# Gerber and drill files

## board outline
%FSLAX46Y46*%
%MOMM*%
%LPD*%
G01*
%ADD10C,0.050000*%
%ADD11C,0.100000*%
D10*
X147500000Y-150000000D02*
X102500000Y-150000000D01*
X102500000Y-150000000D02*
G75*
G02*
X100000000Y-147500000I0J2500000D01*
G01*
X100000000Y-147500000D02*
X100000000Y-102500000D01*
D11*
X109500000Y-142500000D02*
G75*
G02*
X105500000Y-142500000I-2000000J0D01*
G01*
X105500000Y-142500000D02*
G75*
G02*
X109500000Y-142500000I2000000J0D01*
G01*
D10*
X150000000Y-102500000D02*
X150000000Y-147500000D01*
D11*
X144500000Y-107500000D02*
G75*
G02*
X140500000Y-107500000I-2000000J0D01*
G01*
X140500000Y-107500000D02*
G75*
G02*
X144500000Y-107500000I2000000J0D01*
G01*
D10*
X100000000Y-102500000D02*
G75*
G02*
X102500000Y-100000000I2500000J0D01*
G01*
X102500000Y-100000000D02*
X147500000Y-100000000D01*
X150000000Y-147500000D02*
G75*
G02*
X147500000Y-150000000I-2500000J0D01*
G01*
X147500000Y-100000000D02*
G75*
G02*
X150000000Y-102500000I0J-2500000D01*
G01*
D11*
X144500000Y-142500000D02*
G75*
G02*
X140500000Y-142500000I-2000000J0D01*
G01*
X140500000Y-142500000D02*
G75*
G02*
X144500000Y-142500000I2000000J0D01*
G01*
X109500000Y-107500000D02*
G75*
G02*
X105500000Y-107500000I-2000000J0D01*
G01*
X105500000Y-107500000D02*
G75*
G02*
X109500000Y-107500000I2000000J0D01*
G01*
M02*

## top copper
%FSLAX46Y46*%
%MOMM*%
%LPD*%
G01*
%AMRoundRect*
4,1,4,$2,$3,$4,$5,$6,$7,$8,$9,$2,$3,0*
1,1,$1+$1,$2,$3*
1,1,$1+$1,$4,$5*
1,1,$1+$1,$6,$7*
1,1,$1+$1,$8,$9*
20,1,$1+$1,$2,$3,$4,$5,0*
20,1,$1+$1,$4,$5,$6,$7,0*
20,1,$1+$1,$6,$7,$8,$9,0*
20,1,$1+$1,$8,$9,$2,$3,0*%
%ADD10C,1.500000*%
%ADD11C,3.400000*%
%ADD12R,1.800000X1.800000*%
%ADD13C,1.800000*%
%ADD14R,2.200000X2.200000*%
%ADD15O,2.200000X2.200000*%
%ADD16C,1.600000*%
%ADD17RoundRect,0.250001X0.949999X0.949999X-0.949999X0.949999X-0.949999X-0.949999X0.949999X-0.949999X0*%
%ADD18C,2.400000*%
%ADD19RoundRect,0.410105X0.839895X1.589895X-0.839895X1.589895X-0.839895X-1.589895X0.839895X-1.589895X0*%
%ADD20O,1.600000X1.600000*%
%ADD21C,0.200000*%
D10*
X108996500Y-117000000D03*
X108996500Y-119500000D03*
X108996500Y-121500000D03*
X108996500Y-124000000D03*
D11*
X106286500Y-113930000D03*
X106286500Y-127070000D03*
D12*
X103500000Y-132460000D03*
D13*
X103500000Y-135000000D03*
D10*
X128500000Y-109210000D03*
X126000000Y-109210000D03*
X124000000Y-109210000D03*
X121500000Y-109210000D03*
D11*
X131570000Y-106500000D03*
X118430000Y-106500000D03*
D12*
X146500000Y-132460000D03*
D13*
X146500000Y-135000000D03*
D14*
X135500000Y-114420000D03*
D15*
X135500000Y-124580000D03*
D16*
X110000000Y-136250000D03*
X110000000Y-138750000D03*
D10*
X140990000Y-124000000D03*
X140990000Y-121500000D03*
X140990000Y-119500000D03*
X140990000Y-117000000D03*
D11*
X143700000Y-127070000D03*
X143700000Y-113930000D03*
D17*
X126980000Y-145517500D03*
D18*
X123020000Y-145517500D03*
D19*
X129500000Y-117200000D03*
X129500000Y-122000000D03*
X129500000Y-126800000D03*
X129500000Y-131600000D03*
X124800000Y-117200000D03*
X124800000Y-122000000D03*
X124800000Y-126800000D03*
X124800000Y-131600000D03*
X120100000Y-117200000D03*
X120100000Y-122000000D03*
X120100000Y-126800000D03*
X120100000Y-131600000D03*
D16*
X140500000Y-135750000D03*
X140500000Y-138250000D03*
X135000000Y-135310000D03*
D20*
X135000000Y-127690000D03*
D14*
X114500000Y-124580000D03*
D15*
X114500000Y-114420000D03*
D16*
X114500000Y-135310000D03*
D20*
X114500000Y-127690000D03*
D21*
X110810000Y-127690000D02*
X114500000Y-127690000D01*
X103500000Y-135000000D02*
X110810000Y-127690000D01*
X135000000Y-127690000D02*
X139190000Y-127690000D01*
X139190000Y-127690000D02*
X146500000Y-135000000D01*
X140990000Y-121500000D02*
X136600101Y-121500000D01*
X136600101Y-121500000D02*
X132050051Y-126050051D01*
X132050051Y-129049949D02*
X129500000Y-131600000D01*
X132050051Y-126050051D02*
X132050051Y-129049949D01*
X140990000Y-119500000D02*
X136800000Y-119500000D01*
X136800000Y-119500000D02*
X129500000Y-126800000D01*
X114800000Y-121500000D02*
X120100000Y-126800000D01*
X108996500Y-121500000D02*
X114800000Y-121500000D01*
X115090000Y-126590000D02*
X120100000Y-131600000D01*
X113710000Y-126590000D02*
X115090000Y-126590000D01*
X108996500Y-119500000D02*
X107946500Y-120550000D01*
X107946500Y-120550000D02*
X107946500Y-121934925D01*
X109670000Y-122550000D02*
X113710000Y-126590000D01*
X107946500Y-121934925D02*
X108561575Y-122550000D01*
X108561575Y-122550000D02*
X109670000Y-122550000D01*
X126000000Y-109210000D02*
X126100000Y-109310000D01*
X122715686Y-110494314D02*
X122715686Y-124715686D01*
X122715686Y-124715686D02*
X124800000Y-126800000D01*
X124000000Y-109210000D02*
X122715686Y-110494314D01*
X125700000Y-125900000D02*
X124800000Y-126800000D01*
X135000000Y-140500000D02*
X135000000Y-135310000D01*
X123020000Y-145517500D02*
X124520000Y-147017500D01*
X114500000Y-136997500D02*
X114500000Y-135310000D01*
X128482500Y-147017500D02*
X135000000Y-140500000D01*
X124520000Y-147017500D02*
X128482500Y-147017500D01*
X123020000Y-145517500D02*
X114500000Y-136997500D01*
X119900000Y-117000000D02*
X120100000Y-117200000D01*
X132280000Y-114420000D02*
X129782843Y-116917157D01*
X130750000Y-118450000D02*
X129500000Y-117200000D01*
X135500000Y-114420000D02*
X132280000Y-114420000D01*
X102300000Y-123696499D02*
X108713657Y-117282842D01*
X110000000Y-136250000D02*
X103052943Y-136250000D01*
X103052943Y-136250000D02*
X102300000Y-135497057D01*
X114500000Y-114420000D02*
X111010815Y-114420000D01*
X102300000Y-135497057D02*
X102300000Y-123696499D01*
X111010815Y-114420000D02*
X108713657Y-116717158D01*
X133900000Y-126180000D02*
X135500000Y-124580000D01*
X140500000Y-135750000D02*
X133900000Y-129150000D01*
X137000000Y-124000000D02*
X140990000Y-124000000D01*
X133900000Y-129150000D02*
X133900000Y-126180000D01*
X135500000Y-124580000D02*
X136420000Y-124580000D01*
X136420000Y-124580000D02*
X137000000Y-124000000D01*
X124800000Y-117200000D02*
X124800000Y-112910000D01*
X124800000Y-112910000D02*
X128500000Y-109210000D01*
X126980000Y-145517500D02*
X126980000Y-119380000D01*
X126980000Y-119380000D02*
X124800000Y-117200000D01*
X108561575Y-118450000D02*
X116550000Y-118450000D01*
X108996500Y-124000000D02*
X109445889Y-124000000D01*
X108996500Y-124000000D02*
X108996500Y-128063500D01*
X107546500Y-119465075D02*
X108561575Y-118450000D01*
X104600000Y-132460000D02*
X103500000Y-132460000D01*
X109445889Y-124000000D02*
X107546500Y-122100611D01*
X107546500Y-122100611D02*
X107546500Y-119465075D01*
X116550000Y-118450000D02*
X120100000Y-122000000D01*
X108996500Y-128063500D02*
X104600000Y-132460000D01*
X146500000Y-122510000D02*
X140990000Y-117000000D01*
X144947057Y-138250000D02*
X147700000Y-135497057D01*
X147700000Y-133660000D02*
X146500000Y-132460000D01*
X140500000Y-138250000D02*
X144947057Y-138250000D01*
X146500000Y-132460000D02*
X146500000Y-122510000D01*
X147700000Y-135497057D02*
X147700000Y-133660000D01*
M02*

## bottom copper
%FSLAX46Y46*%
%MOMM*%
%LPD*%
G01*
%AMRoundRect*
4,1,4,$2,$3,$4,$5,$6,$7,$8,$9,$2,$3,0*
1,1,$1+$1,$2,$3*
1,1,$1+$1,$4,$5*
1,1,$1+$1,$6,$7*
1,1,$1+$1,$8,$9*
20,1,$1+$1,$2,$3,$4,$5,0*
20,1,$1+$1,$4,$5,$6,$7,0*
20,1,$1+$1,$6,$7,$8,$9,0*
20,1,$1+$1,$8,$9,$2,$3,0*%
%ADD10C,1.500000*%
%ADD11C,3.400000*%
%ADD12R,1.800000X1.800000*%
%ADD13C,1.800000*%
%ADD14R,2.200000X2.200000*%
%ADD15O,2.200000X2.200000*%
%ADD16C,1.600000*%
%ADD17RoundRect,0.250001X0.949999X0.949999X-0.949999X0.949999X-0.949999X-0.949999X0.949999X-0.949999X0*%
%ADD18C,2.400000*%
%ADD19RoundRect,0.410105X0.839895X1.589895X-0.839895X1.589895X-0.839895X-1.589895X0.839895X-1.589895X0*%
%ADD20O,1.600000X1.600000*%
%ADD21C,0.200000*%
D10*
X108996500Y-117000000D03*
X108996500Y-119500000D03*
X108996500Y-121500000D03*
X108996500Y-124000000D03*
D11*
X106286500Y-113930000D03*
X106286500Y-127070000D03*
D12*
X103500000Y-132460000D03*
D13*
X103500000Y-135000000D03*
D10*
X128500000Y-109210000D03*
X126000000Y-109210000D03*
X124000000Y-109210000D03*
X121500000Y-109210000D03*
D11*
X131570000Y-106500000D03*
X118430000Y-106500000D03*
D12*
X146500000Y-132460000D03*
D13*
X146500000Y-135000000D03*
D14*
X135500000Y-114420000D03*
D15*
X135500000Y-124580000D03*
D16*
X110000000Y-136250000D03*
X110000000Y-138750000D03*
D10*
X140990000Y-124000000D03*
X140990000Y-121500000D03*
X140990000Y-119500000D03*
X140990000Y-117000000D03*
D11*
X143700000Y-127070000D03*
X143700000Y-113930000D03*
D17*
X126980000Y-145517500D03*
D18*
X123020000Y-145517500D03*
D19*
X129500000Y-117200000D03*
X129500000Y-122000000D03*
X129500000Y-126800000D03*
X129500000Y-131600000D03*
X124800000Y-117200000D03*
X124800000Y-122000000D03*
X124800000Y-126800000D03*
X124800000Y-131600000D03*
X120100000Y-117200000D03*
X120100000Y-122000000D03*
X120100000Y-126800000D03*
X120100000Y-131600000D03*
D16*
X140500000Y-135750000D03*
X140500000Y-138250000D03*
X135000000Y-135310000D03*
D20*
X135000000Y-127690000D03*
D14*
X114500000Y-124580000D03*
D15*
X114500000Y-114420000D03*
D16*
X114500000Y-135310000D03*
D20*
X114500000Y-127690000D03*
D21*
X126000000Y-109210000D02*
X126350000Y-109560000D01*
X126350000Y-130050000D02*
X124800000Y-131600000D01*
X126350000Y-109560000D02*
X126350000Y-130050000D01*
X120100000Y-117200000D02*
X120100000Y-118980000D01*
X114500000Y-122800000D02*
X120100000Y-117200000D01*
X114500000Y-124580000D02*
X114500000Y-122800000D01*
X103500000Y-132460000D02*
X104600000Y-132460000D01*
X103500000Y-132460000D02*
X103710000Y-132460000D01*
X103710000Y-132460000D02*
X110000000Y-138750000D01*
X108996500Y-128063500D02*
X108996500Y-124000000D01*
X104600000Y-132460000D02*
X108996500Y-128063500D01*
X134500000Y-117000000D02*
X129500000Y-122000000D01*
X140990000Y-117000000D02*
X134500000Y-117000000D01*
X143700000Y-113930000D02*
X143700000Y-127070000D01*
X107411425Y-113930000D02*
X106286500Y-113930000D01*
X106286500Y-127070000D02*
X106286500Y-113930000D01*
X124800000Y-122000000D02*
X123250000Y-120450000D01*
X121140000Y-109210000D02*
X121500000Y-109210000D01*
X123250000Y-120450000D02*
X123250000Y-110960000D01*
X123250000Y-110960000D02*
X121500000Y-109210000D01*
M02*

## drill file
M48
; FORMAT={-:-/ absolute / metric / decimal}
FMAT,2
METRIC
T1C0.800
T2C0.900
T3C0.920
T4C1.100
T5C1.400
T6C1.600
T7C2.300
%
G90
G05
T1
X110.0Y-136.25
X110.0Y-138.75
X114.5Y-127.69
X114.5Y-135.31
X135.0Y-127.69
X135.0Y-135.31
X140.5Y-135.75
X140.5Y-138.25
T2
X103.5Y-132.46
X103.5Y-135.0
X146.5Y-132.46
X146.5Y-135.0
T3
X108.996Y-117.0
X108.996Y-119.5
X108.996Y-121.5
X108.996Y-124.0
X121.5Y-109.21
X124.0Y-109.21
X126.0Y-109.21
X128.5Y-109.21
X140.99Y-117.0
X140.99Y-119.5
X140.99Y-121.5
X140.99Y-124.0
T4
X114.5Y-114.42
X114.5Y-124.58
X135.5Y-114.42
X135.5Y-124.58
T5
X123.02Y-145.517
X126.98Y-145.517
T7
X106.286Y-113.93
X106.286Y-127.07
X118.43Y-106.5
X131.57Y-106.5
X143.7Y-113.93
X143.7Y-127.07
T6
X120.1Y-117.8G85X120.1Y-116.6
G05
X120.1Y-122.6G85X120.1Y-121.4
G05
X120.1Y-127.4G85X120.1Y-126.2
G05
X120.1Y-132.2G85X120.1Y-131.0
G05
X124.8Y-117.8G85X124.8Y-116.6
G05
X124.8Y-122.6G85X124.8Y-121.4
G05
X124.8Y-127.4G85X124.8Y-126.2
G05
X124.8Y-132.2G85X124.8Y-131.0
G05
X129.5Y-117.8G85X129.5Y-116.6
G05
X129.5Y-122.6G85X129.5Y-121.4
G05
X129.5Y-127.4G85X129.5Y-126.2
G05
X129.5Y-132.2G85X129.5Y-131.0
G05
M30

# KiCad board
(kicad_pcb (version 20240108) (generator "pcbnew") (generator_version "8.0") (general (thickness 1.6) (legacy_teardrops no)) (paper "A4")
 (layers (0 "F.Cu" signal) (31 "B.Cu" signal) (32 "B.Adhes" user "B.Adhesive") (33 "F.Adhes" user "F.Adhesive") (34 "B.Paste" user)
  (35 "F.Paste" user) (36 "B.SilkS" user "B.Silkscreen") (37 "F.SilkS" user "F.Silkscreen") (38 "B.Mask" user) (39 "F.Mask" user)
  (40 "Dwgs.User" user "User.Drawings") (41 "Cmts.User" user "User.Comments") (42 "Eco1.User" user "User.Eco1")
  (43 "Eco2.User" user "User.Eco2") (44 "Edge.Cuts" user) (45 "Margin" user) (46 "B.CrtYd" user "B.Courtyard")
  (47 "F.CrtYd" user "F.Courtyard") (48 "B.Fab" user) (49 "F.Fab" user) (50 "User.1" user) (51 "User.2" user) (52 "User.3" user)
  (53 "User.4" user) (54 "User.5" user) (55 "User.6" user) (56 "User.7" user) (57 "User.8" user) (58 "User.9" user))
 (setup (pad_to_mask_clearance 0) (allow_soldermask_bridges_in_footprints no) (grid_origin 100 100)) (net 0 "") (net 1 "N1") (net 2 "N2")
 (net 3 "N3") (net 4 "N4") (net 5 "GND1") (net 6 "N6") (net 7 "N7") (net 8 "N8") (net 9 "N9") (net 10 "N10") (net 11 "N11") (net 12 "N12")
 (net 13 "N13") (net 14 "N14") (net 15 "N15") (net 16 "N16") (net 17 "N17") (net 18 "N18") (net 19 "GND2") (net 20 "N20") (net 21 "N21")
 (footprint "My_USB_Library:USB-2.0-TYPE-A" (layer "F.Cu") (at 95.9865 120.5 -90)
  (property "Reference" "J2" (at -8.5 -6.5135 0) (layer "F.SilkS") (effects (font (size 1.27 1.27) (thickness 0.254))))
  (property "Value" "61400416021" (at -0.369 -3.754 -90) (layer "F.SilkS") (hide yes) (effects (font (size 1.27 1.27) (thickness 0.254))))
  (pad "1" thru_hole circle (at -3.5 -13.01) (size 1.5 1.5) (drill 0.92) (layers "*.Cu" "*.Mask" "F.SilkS") (remove_unused_layers no)
   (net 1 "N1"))
  (pad "2" thru_hole circle (at -1 -13.01) (size 1.5 1.5) (drill 0.92) (layers "*.Cu" "*.Mask" "F.SilkS") (remove_unused_layers no)
   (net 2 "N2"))
  (pad "3" thru_hole circle (at 1 -13.01) (size 1.5 1.5) (drill 0.92) (layers "*.Cu" "*.Mask" "F.SilkS") (remove_unused_layers no)
   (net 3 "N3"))
  (pad "4" thru_hole circle (at 3.5 -13.01) (size 1.5 1.5) (drill 0.92) (layers "*.Cu" "*.Mask" "F.SilkS") (remove_unused_layers no)
   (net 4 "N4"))
  (pad "5" thru_hole circle (at -6.57 -10.3) (size 3.4 3.4) (drill 2.3) (layers "*.Cu" "*.Mask" "F.SilkS") (remove_unused_layers no)
   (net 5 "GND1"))
  (pad "6" thru_hole circle (at 6.57 -10.3) (size 3.4 3.4) (drill 2.3) (layers "*.Cu" "*.Mask" "F.SilkS") (remove_unused_layers no)
   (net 5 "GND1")))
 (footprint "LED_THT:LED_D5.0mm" (layer "F.Cu") (at 103.5 132.46 -90)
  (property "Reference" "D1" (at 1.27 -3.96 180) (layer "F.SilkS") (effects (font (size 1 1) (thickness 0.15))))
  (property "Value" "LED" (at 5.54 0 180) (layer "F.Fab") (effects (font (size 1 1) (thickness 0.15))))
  (pad "1" thru_hole rect (at 0 0 270) (size 1.8 1.8) (drill 0.9) (layers "*.Cu" "*.Mask") (remove_unused_layers no) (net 4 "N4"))
  (pad "2" thru_hole circle (at 2.54 0 270) (size 1.8 1.8) (drill 0.9) (layers "*.Cu" "*.Mask") (remove_unused_layers no) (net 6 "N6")))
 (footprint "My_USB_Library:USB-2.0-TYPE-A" (layer "F.Cu") (at 125 96.2 180)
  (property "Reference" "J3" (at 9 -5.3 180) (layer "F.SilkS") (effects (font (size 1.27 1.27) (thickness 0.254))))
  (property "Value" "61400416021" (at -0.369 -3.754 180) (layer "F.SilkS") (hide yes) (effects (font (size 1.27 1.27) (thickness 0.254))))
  (pad "1" thru_hole circle (at -3.5 -13.01 270) (size 1.5 1.5) (drill 0.92) (layers "*.Cu" "*.Mask" "F.SilkS") (remove_unused_layers no)
   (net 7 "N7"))
  (pad "2" thru_hole circle (at -1 -13.01 270) (size 1.5 1.5) (drill 0.92) (layers "*.Cu" "*.Mask" "F.SilkS") (remove_unused_layers no)
   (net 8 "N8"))
  (pad "3" thru_hole circle (at 1 -13.01 270) (size 1.5 1.5) (drill 0.92) (layers "*.Cu" "*.Mask" "F.SilkS") (remove_unused_layers no)
   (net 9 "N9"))
  (pad "4" thru_hole circle (at 3.5 -13.01 270) (size 1.5 1.5) (drill 0.92) (layers "*.Cu" "*.Mask" "F.SilkS") (remove_unused_layers no)
   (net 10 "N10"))
  (pad "5" thru_hole circle (at -6.57 -10.3 270) (size 3.4 3.4) (drill 2.3) (layers "*.Cu" "*.Mask" "F.SilkS") (remove_unused_layers no)
   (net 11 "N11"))
  (pad "6" thru_hole circle (at 6.57 -10.3 270) (size 3.4 3.4) (drill 2.3) (layers "*.Cu" "*.Mask" "F.SilkS") (remove_unused_layers no)
   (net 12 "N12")))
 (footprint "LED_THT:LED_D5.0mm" (layer "F.Cu") (at 146.5 132.46 -90)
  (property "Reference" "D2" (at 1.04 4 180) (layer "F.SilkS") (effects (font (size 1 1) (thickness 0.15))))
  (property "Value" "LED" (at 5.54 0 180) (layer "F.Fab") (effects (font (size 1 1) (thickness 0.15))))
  (pad "1" thru_hole rect (at 0 0 270) (size 1.8 1.8) (drill 0.9) (layers "*.Cu" "*.Mask") (remove_unused_layers no) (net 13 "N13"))
  (pad "2" thru_hole circle (at 2.54 0 270) (size 1.8 1.8) (drill 0.9) (layers "*.Cu" "*.Mask") (remove_unused_layers no) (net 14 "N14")))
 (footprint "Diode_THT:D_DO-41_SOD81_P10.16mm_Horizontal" (layer "F.Cu") (at 135.5 114.42 -90)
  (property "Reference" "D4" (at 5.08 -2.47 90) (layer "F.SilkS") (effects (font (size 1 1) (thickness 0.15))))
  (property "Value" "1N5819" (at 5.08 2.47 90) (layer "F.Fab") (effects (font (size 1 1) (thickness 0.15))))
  (pad "1" thru_hole rect (at 0 0 270) (size 2.2 2.2) (drill 1.1) (layers "*.Cu" "*.Mask") (remove_unused_layers no) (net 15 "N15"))
  (pad "2" thru_hole oval (at 10.16 0 270) (size 2.2 2.2) (drill 1.1) (layers "*.Cu" "*.Mask") (remove_unused_layers no) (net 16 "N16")))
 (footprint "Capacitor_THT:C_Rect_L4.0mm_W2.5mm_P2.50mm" (layer "F.Cu") (at 110 136.25 -90)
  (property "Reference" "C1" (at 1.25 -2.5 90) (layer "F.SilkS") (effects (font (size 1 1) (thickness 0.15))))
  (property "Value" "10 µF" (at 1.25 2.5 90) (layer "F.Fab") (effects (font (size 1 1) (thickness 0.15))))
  (pad "1" thru_hole circle (at 0 0 270) (size 1.6 1.6) (drill 0.8) (layers "*.Cu" "*.Mask") (remove_unused_layers no) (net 1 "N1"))
  (pad "2" thru_hole circle (at 2.5 0 270) (size 1.6 1.6) (drill 0.8) (layers "*.Cu" "*.Mask") (remove_unused_layers no) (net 4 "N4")))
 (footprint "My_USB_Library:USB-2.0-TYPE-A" (layer "F.Cu") (at 154 120.5 90)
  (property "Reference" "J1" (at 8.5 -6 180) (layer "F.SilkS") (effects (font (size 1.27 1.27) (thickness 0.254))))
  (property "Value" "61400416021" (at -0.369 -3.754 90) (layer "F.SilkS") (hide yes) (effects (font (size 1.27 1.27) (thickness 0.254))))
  (pad "1" thru_hole circle (at -3.5 -13.01 180) (size 1.5 1.5) (drill 0.92) (layers "*.Cu" "*.Mask" "F.SilkS") (remove_unused_layers no)
   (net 16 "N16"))
  (pad "2" thru_hole circle (at -1 -13.01 180) (size 1.5 1.5) (drill 0.92) (layers "*.Cu" "*.Mask" "F.SilkS") (remove_unused_layers no)
   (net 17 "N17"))
  (pad "3" thru_hole circle (at 1 -13.01 180) (size 1.5 1.5) (drill 0.92) (layers "*.Cu" "*.Mask" "F.SilkS") (remove_unused_layers no)
   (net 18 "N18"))
  (pad "4" thru_hole circle (at 3.5 -13.01 180) (size 1.5 1.5) (drill 0.92) (layers "*.Cu" "*.Mask" "F.SilkS") (remove_unused_layers no)
   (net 13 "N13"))
  (pad "5" thru_hole circle (at -6.57 -10.3 180) (size 3.4 3.4) (drill 2.3) (layers "*.Cu" "*.Mask" "F.SilkS") (remove_unused_layers no)
   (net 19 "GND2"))
  (pad "6" thru_hole circle (at 6.57 -10.3 180) (size 3.4 3.4) (drill 2.3) (layers "*.Cu" "*.Mask" "F.SilkS") (remove_unused_layers no)
   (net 19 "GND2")))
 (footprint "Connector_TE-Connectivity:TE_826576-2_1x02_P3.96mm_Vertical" (layer "F.Cu") (at 126.98 145.5175 180)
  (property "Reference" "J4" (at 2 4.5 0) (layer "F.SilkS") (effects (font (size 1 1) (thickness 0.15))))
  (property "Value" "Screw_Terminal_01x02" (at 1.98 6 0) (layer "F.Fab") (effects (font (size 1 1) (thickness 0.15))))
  (pad "1" thru_hole roundrect (at 0 0 180) (size 2.4 2.4) (drill 1.4) (layers "*.Cu" "*.Mask") (remove_unused_layers no)
   (roundrect_rratio 0.104167) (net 7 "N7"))
  (pad "2" thru_hole circle (at 3.96 0 180) (size 2.4 2.4) (drill 1.4) (layers "*.Cu" "*.Mask") (remove_unused_layers no) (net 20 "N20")))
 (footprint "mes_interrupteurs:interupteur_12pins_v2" (layer "F.Cu") (at 129.5 117.2 180)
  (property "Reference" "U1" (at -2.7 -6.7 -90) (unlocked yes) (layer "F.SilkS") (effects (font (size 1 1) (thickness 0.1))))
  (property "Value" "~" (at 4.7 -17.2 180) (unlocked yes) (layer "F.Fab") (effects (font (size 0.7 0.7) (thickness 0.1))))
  (pad "1" thru_hole roundrect (at 0 0 180) (size 2.5 4) (drill oval 1.6 2.8) (layers "*.Cu" "*.Mask") (remove_unused_layers no)
   (roundrect_rratio 0.1640419948) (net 15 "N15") (thermal_bridge_angle 45))
  (pad "2" thru_hole roundrect (at 0 -4.8 180) (size 2.5 4) (drill oval 1.6 2.8) (layers "*.Cu" "*.Mask") (remove_unused_layers no)
   (roundrect_rratio 0.1640419948) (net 13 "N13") (thermal_bridge_angle 45))
  (pad "3" thru_hole roundrect (at 0 -9.6 180) (size 2.5 4) (drill oval 1.6 2.8) (layers "*.Cu" "*.Mask") (remove_unused_layers no)
   (roundrect_rratio 0.1640419948) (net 18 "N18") (thermal_bridge_angle 45))
  (pad "4" thru_hole roundrect (at 0 -14.4 180) (size 2.5 4) (drill oval 1.6 2.8) (layers "*.Cu" "*.Mask") (remove_unused_layers no)
   (roundrect_rratio 0.1640419948) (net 17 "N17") (thermal_bridge_angle 45))
  (pad "5" thru_hole roundrect (at 4.7 0 180) (size 2.5 4) (drill oval 1.6 2.8) (layers "*.Cu" "*.Mask") (remove_unused_layers no)
   (roundrect_rratio 0.1640419948) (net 7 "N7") (thermal_bridge_angle 45))
  (pad "6" thru_hole roundrect (at 4.7 -4.8 180) (size 2.5 4) (drill oval 1.6 2.8) (layers "*.Cu" "*.Mask") (remove_unused_layers no)
   (roundrect_rratio 0.1640419948) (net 10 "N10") (thermal_bridge_angle 45))
  (pad "7" thru_hole roundrect (at 4.7 -9.6 180) (size 2.5 4) (drill oval 1.6 2.8) (layers "*.Cu" "*.Mask") (remove_unused_layers no)
   (roundrect_rratio 0.1640419948) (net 9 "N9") (thermal_bridge_angle 45))
  (pad "8" thru_hole roundrect (at 4.7 -14.4 180) (size 2.5 4) (drill oval 1.6 2.8) (layers "*.Cu" "*.Mask") (remove_unused_layers no)
   (roundrect_rratio 0.1640419948) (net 8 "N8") (thermal_bridge_angle 45))
  (pad "9" thru_hole roundrect (at 9.4 0 180) (size 2.5 4) (drill oval 1.6 2.8) (layers "*.Cu" "*.Mask") (remove_unused_layers no)
   (roundrect_rratio 0.1640419948) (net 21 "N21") (thermal_bridge_angle 45))
  (pad "10" thru_hole roundrect (at 9.4 -4.8 180) (size 2.5 4) (drill oval 1.6 2.8) (layers "*.Cu" "*.Mask") (remove_unused_layers no)
   (roundrect_rratio 0.1640419948) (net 4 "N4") (thermal_bridge_angle 45))
  (pad "11" thru_hole roundrect (at 9.4 -9.6 180) (size 2.5 4) (drill oval 1.6 2.8) (layers "*.Cu" "*.Mask") (remove_unused_layers no)
   (roundrect_rratio 0.1640419948) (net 3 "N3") (thermal_bridge_angle 45))
  (pad "12" thru_hole roundrect (at 9.4 -14.4 180) (size 2.5 4) (drill oval 1.6 2.8) (layers "*.Cu" "*.Mask") (remove_unused_layers no)
   (roundrect_rratio 0.1640419948) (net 2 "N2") (thermal_bridge_angle 45)))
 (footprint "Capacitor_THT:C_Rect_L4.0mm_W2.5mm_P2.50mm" (layer "F.Cu") (at 140.5 135.75 -90)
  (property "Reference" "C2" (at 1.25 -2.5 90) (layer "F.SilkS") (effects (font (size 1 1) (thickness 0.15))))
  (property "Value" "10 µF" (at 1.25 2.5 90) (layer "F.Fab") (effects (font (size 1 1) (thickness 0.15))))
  (pad "1" thru_hole circle (at 0 0 270) (size 1.6 1.6) (drill 0.8) (layers "*.Cu" "*.Mask") (remove_unused_layers no) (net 16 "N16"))
  (pad "2" thru_hole circle (at 2.5 0 270) (size 1.6 1.6) (drill 0.8) (layers "*.Cu" "*.Mask") (remove_unused_layers no) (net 13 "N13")))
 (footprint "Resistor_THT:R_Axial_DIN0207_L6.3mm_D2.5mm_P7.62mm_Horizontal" (layer "F.Cu") (at 135 135.31 90)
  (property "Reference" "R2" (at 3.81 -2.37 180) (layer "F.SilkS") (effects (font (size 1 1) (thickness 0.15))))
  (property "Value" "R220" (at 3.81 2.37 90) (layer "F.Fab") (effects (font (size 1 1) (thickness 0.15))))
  (pad "1" thru_hole circle (at 0 0 90) (size 1.6 1.6) (drill 0.8) (layers "*.Cu" "*.Mask") (remove_unused_layers no) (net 20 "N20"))
  (pad "2" thru_hole oval (at 7.62 0 90) (size 1.6 1.6) (drill 0.8) (layers "*.Cu" "*.Mask") (remove_unused_layers no) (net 14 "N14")))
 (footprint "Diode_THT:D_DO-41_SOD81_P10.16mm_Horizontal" (layer "F.Cu") (at 114.5 124.58 90)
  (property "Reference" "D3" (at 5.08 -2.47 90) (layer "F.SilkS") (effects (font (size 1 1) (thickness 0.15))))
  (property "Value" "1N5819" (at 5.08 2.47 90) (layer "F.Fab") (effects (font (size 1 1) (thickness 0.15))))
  (pad "1" thru_hole rect (at 0 0 90) (size 2.2 2.2) (drill 1.1) (layers "*.Cu" "*.Mask") (remove_unused_layers no) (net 21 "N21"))
  (pad "2" thru_hole oval (at 10.16 0 90) (size 2.2 2.2) (drill 1.1) (layers "*.Cu" "*.Mask") (remove_unused_layers no) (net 1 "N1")))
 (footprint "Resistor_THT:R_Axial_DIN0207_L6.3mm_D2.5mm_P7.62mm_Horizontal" (layer "F.Cu") (at 114.5 135.31 90)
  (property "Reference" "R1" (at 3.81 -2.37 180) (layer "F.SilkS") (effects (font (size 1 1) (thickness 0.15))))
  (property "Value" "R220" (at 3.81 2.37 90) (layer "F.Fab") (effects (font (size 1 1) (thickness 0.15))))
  (pad "1" thru_hole circle (at 0 0 90) (size 1.6 1.6) (drill 0.8) (layers "*.Cu" "*.Mask") (remove_unused_layers no) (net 20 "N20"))
  (pad "2" thru_hole oval (at 7.62 0 90) (size 1.6 1.6) (drill 0.8) (layers "*.Cu" "*.Mask") (remove_unused_layers no) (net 6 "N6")))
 (gr_line (start 147.5 150) (end 102.5 150) (stroke (width 0.05) (type default)) (layer "Edge.Cuts"))
 (gr_arc (start 102.5 150) (mid 100.732233 149.267767) (end 100 147.5) (stroke (width 0.05) (type default)) (layer "Edge.Cuts"))
 (gr_line (start 100 147.5) (end 100 102.5) (stroke (width 0.05) (type default)) (layer "Edge.Cuts"))
 (gr_circle (center 107.5 142.5) (end 109.5 142.5) (stroke (width 0.1) (type default)) (fill none) (layer "Edge.Cuts"))
 (gr_line (start 150 102.5) (end 150 147.5) (stroke (width 0.05) (type default)) (layer "Edge.Cuts"))
 (gr_circle (center 142.5 107.5) (end 144.5 107.5) (stroke (width 0.1) (type default)) (fill none) (layer "Edge.Cuts"))
 (gr_arc (start 100 102.5) (mid 100.732233 100.732233) (end 102.5 100) (stroke (width 0.05) (type default)) (layer "Edge.Cuts"))
 (gr_line (start 102.5 100) (end 147.5 100) (stroke (width 0.05) (type default)) (layer "Edge.Cuts"))
 (gr_arc (start 150 147.5) (mid 149.267767 149.267767) (end 147.5 150) (stroke (width 0.05) (type default)) (layer "Edge.Cuts"))
 (gr_arc (start 147.5 100) (mid 149.267767 100.732233) (end 150 102.5) (stroke (width 0.05) (type default)) (layer "Edge.Cuts"))
 (gr_circle (center 142.5 142.5) (end 144.5 142.5) (stroke (width 0.1) (type default)) (fill none) (layer "Edge.Cuts"))
 (gr_circle (center 107.5 107.5) (end 109.5 107.5) (stroke (width 0.1) (type default)) (fill none) (layer "Edge.Cuts"))
 (segment (start 110.81 127.69) (end 114.5 127.69) (width 0.2) (layer "F.Cu") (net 6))
 (segment (start 103.5 135) (end 110.81 127.69) (width 0.2) (layer "F.Cu") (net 6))
 (segment (start 135 127.69) (end 139.19 127.69) (width 0.2) (layer "F.Cu") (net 14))
 (segment (start 139.19 127.69) (end 146.5 135) (width 0.2) (layer "F.Cu") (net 14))
 (segment (start 140.99 121.5) (end 136.600101 121.5) (width 0.2) (layer "F.Cu") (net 17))
 (segment (start 136.600101 121.5) (end 132.050051 126.050051) (width 0.2) (layer "F.Cu") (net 17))
 (segment (start 132.050051 129.049949) (end 129.5 131.6) (width 0.2) (layer "F.Cu") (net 17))
 (segment (start 132.050051 126.050051) (end 132.050051 129.049949) (width 0.2) (layer "F.Cu") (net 17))
 (segment (start 140.99 119.5) (end 136.8 119.5) (width 0.2) (layer "F.Cu") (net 18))
 (segment (start 136.8 119.5) (end 129.5 126.8) (width 0.2) (layer "F.Cu") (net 18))
 (segment (start 114.8 121.5) (end 120.1 126.8) (width 0.2) (layer "F.Cu") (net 3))
 (segment (start 108.9965 121.5) (end 114.8 121.5) (width 0.2) (layer "F.Cu") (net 3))
 (segment (start 115.09 126.59) (end 120.1 131.6) (width 0.2) (layer "F.Cu") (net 2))
 (segment (start 113.71 126.59) (end 115.09 126.59) (width 0.2) (layer "F.Cu") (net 2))
 (segment (start 108.9965 119.5) (end 107.9465 120.55) (width 0.2) (layer "F.Cu") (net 2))
 (segment (start 107.9465 120.55) (end 107.9465 121.934925) (width 0.2) (layer "F.Cu") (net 2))
 (segment (start 109.67 122.55) (end 113.71 126.59) (width 0.2) (layer "F.Cu") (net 2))
 (segment (start 107.9465 121.934925) (end 108.561575 122.55) (width 0.2) (layer "F.Cu") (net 2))
 (segment (start 108.561575 122.55) (end 109.67 122.55) (width 0.2) (layer "F.Cu") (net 2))
 (segment (start 126 109.21) (end 126.1 109.31) (width 0.2) (layer "F.Cu") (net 8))
 (segment (start 126 109.21) (end 126.35 109.56) (width 0.2) (layer "B.Cu") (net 8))
 (segment (start 126.35 130.05) (end 124.8 131.6) (width 0.2) (layer "B.Cu") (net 8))
 (segment (start 126.35 109.56) (end 126.35 130.05) (width 0.2) (layer "B.Cu") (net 8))
 (segment (start 122.715686 110.494314) (end 122.715686 124.715686) (width 0.2) (layer "F.Cu") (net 9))
 (segment (start 122.715686 124.715686) (end 124.8 126.8) (width 0.2) (layer "F.Cu") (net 9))
 (segment (start 124 109.21) (end 122.715686 110.494314) (width 0.2) (layer "F.Cu") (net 9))
 (segment (start 125.7 125.9) (end 124.8 126.8) (width 0.2) (layer "F.Cu") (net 9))
 (segment (start 135 140.5) (end 135 135.31) (width 0.2) (layer "F.Cu") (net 20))
 (segment (start 123.02 145.5175) (end 124.52 147.0175) (width 0.2) (layer "F.Cu") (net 20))
 (segment (start 114.5 136.9975) (end 114.5 135.31) (width 0.2) (layer "F.Cu") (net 20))
 (segment (start 128.4825 147.0175) (end 135 140.5) (width 0.2) (layer "F.Cu") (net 20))
 (segment (start 124.52 147.0175) (end 128.4825 147.0175) (width 0.2) (layer "F.Cu") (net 20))
 (segment (start 123.02 145.5175) (end 114.5 136.9975) (width 0.2) (layer "F.Cu") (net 20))
 (segment (start 119.9 117) (end 120.1 117.2) (width 0.2) (layer "F.Cu") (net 21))
 (segment (start 120.1 117.2) (end 120.1 118.98) (width 0.2) (layer "B.Cu") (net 21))
 (segment (start 114.5 122.8) (end 120.1 117.2) (width 0.2) (layer "B.Cu") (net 21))
 (segment (start 114.5 124.58) (end 114.5 122.8) (width 0.2) (layer "B.Cu") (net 21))
 (segment (start 132.28 114.42) (end 129.782843 116.917157) (width 0.2) (layer "F.Cu") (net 15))
 (segment (start 130.75 118.45) (end 129.5 117.2) (width 0.2) (layer "F.Cu") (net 15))
 (segment (start 135.5 114.42) (end 132.28 114.42) (width 0.2) (layer "F.Cu") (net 15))
 (segment (start 102.3 123.696499) (end 108.713657 117.282842) (width 0.2) (layer "F.Cu") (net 1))
 (segment (start 110 136.25) (end 103.052943 136.25) (width 0.2) (layer "F.Cu") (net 1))
 (segment (start 103.052943 136.25) (end 102.3 135.497057) (width 0.2) (layer "F.Cu") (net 1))
 (segment (start 114.5 114.42) (end 111.010815 114.42) (width 0.2) (layer "F.Cu") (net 1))
 (segment (start 102.3 135.497057) (end 102.3 123.696499) (width 0.2) (layer "F.Cu") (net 1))
 (segment (start 111.010815 114.42) (end 108.713657 116.717158) (width 0.2) (layer "F.Cu") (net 1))
 (segment (start 133.9 126.18) (end 135.5 124.58) (width 0.2) (layer "F.Cu") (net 16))
 (segment (start 140.5 135.75) (end 133.9 129.15) (width 0.2) (layer "F.Cu") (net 16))
 (segment (start 137 124) (end 140.99 124) (width 0.2) (layer "F.Cu") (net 16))
 (segment (start 133.9 129.15) (end 133.9 126.18) (width 0.2) (layer "F.Cu") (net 16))
 (segment (start 135.5 124.58) (end 136.42 124.58) (width 0.2) (layer "F.Cu") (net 16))
 (segment (start 136.42 124.58) (end 137 124) (width 0.2) (layer "F.Cu") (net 16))
 (segment (start 124.8 117.2) (end 124.8 112.91) (width 0.2) (layer "F.Cu") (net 7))
 (segment (start 124.8 112.91) (end 128.5 109.21) (width 0.2) (layer "F.Cu") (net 7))
 (segment (start 126.98 145.5175) (end 126.98 119.38) (width 0.2) (layer "F.Cu") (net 7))
 (segment (start 126.98 119.38) (end 124.8 117.2) (width 0.2) (layer "F.Cu") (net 7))
 (segment (start 108.561575 118.45) (end 116.55 118.45) (width 0.2) (layer "F.Cu") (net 4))
 (segment (start 108.9965 124) (end 109.445889 124) (width 0.2) (layer "F.Cu") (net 4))
 (segment (start 108.9965 124) (end 108.9965 128.0635) (width 0.2) (layer "F.Cu") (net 4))
 (segment (start 107.5465 119.465075) (end 108.561575 118.45) (width 0.2) (layer "F.Cu") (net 4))
 (segment (start 104.6 132.46) (end 103.5 132.46) (width 0.2) (layer "F.Cu") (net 4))
 (segment (start 109.445889 124) (end 107.5465 122.100611) (width 0.2) (layer "F.Cu") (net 4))
 (segment (start 107.5465 122.100611) (end 107.5465 119.465075) (width 0.2) (layer "F.Cu") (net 4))
 (segment (start 116.55 118.45) (end 120.1 122) (width 0.2) (layer "F.Cu") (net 4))
 (segment (start 108.9965 128.0635) (end 104.6 132.46) (width 0.2) (layer "F.Cu") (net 4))
 (segment (start 103.5 132.46) (end 104.6 132.46) (width 0.2) (layer "B.Cu") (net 4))
 (segment (start 103.5 132.46) (end 103.71 132.46) (width 0.2) (layer "B.Cu") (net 4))
 (segment (start 103.71 132.46) (end 110 138.75) (width 0.2) (layer "B.Cu") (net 4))
 (segment (start 108.9965 128.0635) (end 108.9965 124) (width 0.2) (layer "B.Cu") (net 4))
 (segment (start 104.6 132.46) (end 108.9965 128.0635) (width 0.2) (layer "B.Cu") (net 4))
 (segment (start 146.5 122.51) (end 140.99 117) (width 0.2) (layer "F.Cu") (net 13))
 (segment (start 144.947057 138.25) (end 147.7 135.497057) (width 0.2) (layer "F.Cu") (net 13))
 (segment (start 147.7 133.66) (end 146.5 132.46) (width 0.2) (layer "F.Cu") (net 13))
 (segment (start 140.5 138.25) (end 144.947057 138.25) (width 0.2) (layer "F.Cu") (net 13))
 (segment (start 146.5 132.46) (end 146.5 122.51) (width 0.2) (layer "F.Cu") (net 13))
 (segment (start 147.7 135.497057) (end 147.7 133.66) (width 0.2) (layer "F.Cu") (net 13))
 (segment (start 134.5 117) (end 129.5 122) (width 0.2) (layer "B.Cu") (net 13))
 (segment (start 140.99 117) (end 134.5 117) (width 0.2) (layer "B.Cu") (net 13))
 (segment (start 143.7 113.93) (end 143.7 127.07) (width 0.2) (layer "B.Cu") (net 19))
 (segment (start 107.411425 113.93) (end 106.2865 113.93) (width 0.2) (layer "B.Cu") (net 5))
 (segment (start 106.2865 127.07) (end 106.2865 113.93) (width 0.2) (layer "B.Cu") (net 5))
 (segment (start 124.8 122) (end 123.25 120.45) (width 0.2) (layer "B.Cu") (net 10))
 (segment (start 121.14 109.21) (end 121.5 109.21) (width 0.2) (layer "B.Cu") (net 10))
 (segment (start 123.25 120.45) (end 123.25 110.96) (width 0.2) (layer "B.Cu") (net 10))
 (segment (start 123.25 110.96) (end 121.5 109.21) (width 0.2) (layer "B.Cu") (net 10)))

